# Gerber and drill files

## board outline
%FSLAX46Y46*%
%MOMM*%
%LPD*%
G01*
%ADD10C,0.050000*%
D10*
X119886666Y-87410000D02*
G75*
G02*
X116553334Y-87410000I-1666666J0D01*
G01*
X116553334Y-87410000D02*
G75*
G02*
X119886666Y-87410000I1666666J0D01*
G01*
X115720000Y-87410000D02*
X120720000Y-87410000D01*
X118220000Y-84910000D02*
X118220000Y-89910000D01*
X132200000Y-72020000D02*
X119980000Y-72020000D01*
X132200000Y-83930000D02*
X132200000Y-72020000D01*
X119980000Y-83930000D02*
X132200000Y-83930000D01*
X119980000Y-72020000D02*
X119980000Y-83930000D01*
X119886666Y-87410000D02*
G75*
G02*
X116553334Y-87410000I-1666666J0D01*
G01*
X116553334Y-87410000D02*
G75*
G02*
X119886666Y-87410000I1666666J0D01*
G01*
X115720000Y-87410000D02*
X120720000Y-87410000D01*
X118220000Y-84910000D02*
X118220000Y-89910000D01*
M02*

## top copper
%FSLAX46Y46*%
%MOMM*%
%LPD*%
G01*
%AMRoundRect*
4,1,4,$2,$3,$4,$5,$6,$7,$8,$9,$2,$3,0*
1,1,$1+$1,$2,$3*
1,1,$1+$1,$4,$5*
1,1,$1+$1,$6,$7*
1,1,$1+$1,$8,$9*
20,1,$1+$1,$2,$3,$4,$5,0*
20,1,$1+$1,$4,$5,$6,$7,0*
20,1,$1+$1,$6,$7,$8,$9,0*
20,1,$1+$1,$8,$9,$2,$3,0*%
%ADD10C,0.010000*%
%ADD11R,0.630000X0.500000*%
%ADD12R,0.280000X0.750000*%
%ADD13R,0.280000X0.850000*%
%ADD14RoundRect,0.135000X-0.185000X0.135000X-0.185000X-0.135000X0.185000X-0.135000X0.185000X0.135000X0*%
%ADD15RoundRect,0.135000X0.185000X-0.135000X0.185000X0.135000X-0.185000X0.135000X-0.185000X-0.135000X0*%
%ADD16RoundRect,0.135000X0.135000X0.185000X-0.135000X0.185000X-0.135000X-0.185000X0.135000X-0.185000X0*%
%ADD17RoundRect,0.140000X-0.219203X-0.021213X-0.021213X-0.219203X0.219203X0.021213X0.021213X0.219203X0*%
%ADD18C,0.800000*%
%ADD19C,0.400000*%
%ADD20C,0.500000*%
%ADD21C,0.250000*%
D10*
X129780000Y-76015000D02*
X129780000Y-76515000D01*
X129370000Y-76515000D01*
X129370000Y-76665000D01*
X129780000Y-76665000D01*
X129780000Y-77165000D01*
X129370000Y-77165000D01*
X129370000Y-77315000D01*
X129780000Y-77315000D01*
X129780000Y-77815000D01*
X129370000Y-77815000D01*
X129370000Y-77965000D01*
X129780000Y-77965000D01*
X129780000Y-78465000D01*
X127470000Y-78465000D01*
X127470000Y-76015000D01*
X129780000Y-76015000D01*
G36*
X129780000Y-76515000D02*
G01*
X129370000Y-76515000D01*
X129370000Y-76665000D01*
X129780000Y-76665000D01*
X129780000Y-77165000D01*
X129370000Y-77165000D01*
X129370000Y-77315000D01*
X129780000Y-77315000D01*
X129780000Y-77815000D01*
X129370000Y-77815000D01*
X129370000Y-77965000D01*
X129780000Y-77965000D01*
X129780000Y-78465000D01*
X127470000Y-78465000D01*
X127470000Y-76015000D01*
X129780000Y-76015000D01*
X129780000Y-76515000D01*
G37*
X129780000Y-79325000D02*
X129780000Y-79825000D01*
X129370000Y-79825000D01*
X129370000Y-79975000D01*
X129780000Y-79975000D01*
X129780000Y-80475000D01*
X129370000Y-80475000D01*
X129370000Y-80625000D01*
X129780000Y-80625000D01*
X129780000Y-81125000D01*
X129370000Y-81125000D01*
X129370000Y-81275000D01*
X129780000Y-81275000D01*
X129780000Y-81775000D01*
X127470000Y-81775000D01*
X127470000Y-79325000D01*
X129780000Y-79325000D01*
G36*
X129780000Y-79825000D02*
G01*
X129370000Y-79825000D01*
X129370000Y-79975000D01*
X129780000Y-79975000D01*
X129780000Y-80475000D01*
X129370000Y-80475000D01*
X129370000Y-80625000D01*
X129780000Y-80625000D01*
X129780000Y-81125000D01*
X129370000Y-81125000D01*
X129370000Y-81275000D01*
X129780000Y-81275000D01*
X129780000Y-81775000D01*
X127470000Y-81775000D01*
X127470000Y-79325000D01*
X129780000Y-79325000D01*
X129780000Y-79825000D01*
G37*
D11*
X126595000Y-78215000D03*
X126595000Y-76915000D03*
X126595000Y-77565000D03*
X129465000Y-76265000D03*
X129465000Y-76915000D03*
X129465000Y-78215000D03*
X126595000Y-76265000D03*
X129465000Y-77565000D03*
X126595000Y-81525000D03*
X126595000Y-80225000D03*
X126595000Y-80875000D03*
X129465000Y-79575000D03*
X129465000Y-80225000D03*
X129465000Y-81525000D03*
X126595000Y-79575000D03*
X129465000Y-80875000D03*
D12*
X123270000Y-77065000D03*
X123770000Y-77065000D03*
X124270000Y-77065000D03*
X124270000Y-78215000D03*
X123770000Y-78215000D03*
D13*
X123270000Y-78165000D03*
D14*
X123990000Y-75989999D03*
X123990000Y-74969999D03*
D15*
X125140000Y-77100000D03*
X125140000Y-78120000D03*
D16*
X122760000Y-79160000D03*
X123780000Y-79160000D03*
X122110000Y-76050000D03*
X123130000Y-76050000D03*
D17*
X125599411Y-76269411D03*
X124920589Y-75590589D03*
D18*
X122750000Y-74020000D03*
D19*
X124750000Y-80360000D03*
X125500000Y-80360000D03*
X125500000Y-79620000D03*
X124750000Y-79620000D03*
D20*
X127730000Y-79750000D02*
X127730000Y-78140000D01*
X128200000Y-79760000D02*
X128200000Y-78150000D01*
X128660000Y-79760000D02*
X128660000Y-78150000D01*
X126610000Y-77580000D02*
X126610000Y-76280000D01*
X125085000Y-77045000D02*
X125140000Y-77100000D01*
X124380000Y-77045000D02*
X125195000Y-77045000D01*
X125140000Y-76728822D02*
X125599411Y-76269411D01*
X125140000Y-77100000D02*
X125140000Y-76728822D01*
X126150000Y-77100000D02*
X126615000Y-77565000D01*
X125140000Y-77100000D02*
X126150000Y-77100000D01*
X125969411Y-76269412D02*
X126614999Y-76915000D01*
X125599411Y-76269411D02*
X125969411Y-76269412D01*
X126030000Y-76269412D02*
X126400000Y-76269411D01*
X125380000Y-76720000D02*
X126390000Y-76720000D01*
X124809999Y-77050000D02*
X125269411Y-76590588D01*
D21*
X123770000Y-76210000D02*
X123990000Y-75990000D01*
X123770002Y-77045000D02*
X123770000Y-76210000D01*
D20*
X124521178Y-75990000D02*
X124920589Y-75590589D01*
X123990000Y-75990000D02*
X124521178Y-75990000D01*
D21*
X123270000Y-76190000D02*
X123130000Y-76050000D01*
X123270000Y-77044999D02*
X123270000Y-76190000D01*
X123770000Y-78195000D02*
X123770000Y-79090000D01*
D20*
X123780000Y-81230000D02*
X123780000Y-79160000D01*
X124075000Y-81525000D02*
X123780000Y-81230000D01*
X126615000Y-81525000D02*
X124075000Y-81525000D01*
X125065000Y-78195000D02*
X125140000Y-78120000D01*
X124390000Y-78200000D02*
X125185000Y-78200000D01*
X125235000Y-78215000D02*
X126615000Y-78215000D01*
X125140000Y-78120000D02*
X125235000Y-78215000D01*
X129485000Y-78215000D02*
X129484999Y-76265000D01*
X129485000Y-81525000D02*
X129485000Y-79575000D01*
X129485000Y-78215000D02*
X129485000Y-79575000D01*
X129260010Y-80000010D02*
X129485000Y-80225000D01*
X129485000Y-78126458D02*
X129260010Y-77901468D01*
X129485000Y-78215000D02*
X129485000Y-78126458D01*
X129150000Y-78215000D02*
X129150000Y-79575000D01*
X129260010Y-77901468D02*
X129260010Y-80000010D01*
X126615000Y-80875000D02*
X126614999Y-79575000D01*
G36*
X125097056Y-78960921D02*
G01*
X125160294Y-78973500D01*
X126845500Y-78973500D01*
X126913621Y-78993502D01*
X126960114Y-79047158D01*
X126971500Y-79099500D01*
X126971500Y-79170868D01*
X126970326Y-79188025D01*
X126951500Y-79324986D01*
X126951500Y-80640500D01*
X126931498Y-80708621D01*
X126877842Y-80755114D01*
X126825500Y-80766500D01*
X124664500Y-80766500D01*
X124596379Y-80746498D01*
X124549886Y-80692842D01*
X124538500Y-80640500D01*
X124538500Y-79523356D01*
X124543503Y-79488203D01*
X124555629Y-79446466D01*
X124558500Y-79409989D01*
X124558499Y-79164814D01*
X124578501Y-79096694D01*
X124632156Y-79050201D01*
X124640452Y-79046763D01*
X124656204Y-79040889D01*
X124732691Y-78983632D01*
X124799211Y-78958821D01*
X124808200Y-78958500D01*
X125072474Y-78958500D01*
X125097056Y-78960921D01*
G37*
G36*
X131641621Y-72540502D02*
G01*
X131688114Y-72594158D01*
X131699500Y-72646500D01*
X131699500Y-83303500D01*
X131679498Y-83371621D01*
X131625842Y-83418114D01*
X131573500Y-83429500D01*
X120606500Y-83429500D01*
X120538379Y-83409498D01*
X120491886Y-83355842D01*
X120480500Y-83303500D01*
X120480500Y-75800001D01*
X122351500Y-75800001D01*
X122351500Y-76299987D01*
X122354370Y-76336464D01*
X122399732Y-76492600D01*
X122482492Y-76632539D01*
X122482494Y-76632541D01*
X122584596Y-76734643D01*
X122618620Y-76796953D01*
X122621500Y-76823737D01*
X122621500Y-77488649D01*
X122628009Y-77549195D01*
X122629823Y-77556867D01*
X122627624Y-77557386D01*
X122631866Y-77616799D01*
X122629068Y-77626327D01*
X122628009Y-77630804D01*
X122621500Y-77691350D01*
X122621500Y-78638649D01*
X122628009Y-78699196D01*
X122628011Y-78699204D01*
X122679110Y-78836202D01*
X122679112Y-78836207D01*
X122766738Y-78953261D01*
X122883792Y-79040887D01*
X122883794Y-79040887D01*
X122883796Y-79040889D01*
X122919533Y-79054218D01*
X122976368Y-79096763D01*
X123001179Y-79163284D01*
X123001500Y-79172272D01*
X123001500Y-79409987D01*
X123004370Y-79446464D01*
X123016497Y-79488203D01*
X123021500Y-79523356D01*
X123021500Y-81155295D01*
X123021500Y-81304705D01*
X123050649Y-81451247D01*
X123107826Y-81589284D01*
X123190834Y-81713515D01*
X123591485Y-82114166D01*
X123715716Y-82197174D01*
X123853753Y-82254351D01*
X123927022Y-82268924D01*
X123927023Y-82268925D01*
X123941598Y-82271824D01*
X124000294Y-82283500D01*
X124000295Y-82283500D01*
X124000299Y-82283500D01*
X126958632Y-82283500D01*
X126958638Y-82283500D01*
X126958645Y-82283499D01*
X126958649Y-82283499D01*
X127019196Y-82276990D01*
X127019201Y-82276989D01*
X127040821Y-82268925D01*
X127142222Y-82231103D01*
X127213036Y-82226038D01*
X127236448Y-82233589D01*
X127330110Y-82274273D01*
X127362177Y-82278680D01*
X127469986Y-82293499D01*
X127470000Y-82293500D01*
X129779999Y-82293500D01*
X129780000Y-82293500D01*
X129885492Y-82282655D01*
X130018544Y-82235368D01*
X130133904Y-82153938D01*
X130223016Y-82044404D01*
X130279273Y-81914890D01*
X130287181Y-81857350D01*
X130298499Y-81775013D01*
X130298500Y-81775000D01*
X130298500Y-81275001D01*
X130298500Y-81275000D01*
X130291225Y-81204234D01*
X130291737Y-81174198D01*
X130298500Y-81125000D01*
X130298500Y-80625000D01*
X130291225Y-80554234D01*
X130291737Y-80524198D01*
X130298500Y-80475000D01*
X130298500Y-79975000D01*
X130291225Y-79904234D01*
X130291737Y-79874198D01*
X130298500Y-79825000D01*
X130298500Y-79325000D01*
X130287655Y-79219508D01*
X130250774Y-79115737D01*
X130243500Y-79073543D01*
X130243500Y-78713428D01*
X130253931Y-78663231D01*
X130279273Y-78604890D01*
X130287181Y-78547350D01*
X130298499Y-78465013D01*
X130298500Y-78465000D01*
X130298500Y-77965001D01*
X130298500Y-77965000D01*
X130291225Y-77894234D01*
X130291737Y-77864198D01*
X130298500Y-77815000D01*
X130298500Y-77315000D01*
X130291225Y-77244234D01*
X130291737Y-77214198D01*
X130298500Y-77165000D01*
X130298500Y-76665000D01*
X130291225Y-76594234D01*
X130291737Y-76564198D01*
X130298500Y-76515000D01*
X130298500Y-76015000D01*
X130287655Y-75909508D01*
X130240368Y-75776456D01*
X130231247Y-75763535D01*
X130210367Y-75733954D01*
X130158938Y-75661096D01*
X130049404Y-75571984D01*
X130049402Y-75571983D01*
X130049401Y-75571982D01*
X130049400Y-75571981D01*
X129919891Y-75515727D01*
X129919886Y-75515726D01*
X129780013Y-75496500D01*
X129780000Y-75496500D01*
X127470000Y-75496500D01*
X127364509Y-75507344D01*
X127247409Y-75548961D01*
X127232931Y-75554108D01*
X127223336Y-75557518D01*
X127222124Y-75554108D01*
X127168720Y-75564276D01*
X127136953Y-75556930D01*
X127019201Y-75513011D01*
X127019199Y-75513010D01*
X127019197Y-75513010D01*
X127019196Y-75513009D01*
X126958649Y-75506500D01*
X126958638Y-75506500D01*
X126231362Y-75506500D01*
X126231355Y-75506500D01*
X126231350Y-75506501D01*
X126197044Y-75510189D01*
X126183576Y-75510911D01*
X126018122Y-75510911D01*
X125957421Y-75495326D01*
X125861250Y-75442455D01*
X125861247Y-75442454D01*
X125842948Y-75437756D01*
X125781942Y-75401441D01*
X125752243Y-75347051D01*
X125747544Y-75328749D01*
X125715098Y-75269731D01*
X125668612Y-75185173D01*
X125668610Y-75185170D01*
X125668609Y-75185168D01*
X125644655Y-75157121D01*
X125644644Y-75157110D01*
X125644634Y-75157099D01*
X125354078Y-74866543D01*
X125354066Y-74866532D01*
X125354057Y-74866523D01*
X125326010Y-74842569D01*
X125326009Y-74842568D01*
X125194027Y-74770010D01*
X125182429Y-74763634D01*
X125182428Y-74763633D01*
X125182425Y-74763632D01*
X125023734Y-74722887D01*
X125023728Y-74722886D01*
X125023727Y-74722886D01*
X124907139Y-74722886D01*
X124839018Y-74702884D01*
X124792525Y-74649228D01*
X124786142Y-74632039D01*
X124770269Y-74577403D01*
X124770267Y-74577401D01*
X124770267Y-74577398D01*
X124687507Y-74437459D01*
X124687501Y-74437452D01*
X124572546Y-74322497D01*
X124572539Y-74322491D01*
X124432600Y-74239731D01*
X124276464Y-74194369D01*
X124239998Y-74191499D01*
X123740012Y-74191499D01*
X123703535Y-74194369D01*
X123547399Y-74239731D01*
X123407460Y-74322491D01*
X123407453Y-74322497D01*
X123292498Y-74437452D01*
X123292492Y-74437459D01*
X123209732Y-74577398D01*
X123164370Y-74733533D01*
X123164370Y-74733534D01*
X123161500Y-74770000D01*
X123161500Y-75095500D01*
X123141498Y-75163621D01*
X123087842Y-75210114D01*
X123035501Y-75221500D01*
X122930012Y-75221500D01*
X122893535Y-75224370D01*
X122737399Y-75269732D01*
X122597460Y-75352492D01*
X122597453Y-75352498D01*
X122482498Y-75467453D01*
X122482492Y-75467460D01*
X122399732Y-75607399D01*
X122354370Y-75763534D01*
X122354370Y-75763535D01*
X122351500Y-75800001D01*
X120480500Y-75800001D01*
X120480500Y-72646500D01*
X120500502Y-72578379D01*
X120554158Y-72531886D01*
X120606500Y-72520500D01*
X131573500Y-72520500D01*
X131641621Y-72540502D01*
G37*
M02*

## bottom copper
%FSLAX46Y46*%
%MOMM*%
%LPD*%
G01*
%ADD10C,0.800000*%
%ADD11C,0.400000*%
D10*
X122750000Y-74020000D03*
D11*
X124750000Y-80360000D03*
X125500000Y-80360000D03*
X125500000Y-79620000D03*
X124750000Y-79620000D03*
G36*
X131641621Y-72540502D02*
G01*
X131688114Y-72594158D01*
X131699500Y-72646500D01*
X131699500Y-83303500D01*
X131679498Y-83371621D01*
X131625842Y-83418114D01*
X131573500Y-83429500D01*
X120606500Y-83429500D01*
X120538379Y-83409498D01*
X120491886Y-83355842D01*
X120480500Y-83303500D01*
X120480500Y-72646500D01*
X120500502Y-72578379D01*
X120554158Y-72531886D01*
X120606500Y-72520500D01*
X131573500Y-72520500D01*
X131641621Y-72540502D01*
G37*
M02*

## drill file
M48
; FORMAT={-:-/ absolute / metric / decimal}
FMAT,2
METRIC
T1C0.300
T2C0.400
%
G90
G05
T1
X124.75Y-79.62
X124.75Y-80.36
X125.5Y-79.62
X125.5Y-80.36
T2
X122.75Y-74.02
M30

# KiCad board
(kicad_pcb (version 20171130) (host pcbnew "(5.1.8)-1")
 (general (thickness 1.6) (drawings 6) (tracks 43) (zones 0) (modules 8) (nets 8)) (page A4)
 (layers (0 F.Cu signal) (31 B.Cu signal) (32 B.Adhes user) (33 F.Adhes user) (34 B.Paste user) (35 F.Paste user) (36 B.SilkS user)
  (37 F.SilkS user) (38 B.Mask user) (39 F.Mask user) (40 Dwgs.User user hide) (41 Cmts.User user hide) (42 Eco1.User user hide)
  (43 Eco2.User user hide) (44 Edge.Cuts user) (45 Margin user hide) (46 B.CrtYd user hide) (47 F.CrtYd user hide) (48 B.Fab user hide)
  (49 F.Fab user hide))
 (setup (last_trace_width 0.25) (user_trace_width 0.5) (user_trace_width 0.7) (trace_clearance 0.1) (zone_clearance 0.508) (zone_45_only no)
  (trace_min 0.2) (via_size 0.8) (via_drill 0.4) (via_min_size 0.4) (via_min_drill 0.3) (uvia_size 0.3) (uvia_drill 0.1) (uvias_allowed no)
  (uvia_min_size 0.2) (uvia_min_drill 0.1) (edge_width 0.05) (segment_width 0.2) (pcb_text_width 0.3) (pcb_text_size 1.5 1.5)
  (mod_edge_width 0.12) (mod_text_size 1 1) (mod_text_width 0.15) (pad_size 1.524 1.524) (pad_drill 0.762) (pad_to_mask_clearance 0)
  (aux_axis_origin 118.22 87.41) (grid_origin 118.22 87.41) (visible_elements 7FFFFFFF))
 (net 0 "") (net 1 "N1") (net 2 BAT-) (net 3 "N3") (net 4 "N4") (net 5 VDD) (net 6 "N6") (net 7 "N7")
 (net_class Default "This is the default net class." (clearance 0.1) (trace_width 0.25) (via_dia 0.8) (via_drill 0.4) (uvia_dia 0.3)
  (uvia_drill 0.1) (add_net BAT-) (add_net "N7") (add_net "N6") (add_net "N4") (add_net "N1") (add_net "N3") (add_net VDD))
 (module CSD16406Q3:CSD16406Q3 (layer F.Cu) (at 128.29 74.07)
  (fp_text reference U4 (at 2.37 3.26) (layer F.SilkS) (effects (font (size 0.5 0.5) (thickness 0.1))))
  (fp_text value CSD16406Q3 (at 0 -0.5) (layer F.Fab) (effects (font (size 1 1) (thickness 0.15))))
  (fp_poly
   (pts (xy 1.49 1.945) (xy 1.49 2.445) (xy 1.08 2.445) (xy 1.08 2.595) (xy 1.49 2.595) (xy 1.49 3.095) (xy 1.08 3.095) (xy 1.08 3.245)
    (xy 1.49 3.245) (xy 1.49 3.745) (xy 1.08 3.745) (xy 1.08 3.895) (xy 1.49 3.895) (xy 1.49 4.395) (xy -0.82 4.395) (xy -0.82 1.945))
   (layer F.Cu) (width 0.01))
  (pad 4 smd rect (at -1.695 4.145) (size 0.63 0.5) (layers F.Cu F.Mask) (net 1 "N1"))
  (pad 2 smd rect (at -1.695 2.845) (size 0.63 0.5) (layers F.Cu F.Mask) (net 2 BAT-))
  (pad 3 smd rect (at -1.695 3.495) (size 0.63 0.5) (layers F.Cu F.Mask) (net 2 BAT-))
  (pad 8 smd rect (at 1.175 2.195) (size 0.63 0.5) (layers F.Cu) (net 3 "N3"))
  (pad 7 smd rect (at 1.175 2.845) (size 0.63 0.5) (layers F.Cu) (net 3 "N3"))
  (pad 5 smd rect (at 1.175 4.145) (size 0.63 0.5) (layers F.Cu) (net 3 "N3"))
  (pad 1 smd rect (at -1.695 2.195) (size 0.63 0.5) (layers F.Cu F.Mask) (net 2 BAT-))
  (pad 6 smd rect (at 1.175 3.495) (size 0.63 0.5) (layers F.Cu) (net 3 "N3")))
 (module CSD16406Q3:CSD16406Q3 (layer F.Cu) (at 128.29 77.38)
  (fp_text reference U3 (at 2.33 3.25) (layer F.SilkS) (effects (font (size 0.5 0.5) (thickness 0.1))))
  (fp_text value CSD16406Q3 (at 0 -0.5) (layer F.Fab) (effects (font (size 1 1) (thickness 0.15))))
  (fp_poly
   (pts (xy 1.49 1.945) (xy 1.49 2.445) (xy 1.08 2.445) (xy 1.08 2.595) (xy 1.49 2.595) (xy 1.49 3.095) (xy 1.08 3.095) (xy 1.08 3.245)
    (xy 1.49 3.245) (xy 1.49 3.745) (xy 1.08 3.745) (xy 1.08 3.895) (xy 1.49 3.895) (xy 1.49 4.395) (xy -0.82 4.395) (xy -0.82 1.945))
   (layer F.Cu) (width 0.01))
  (pad 4 smd rect (at -1.695 4.145) (size 0.63 0.5) (layers F.Cu F.Mask) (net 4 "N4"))
  (pad 2 smd rect (at -1.695 2.845) (size 0.63 0.5) (layers F.Cu F.Mask) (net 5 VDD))
  (pad 3 smd rect (at -1.695 3.495) (size 0.63 0.5) (layers F.Cu F.Mask) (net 5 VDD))
  (pad 8 smd rect (at 1.175 2.195) (size 0.63 0.5) (layers F.Cu) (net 3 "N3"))
  (pad 7 smd rect (at 1.175 2.845) (size 0.63 0.5) (layers F.Cu) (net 3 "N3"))
  (pad 5 smd rect (at 1.175 4.145) (size 0.63 0.5) (layers F.Cu) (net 3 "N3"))
  (pad 1 smd rect (at -1.695 2.195) (size 0.63 0.5) (layers F.Cu F.Mask) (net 5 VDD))
  (pad 6 smd rect (at 1.175 3.495) (size 0.63 0.5) (layers F.Cu) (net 3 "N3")))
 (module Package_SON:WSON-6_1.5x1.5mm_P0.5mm (layer F.Cu) (at 123.77 77.64 90)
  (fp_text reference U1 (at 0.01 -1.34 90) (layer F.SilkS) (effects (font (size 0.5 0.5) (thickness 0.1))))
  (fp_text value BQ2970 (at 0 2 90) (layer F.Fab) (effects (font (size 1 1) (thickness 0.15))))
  (pad 6 smd rect (at 0.575 -0.5) (size 0.28 0.75) (layers F.Cu F.Paste F.Mask) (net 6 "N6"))
  (pad 5 smd rect (at 0.575 0) (size 0.28 0.75) (layers F.Cu F.Paste F.Mask) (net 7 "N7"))
  (pad 4 smd rect (at 0.575 0.5) (size 0.28 0.75) (layers F.Cu F.Paste F.Mask) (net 2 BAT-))
  (pad 3 smd rect (at -0.575 0.5) (size 0.28 0.75) (layers F.Cu F.Paste F.Mask) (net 1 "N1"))
  (pad 2 smd rect (at -0.575 0) (size 0.28 0.75) (layers F.Cu F.Paste F.Mask) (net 4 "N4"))
  (pad 1 smd rect (at -0.525 -0.5) (size 0.28 0.85) (layers F.Cu F.Paste F.Mask)))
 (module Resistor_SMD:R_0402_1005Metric (layer F.Cu) (at 123.99 75.479999 270)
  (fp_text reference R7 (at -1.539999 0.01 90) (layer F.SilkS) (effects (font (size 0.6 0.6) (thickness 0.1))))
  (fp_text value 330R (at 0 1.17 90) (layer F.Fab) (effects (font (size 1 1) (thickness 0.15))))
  (pad 2 smd roundrect (at 0.51 0 270) (size 0.54 0.64) (layers F.Cu F.Paste F.Mask) (roundrect_rratio 0.25) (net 7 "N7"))
  (pad 1 smd roundrect (at -0.51 0 270) (size 0.54 0.64) (layers F.Cu F.Paste F.Mask) (roundrect_rratio 0.25)))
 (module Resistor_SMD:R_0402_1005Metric (layer F.Cu) (at 125.14 77.61 90)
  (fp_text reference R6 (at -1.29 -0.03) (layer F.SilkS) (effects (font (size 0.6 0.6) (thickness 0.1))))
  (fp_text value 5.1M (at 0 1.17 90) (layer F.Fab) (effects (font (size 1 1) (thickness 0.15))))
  (pad 2 smd roundrect (at 0.51 0 90) (size 0.54 0.64) (layers F.Cu F.Paste F.Mask) (roundrect_rratio 0.25) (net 2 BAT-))
  (pad 1 smd roundrect (at -0.51 0 90) (size 0.54 0.64) (layers F.Cu F.Paste F.Mask) (roundrect_rratio 0.25) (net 1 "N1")))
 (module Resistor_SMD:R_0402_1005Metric (layer F.Cu) (at 123.27 79.16 180)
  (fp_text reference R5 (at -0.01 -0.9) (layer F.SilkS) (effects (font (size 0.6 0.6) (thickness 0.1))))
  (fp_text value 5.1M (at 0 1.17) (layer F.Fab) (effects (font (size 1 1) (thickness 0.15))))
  (pad 2 smd roundrect (at 0.51 0 180) (size 0.54 0.64) (layers F.Cu F.Paste F.Mask) (roundrect_rratio 0.25) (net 5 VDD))
  (pad 1 smd roundrect (at -0.51 0 180) (size 0.54 0.64) (layers F.Cu F.Paste F.Mask) (roundrect_rratio 0.25) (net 4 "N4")))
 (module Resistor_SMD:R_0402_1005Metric (layer F.Cu) (at 122.62 76.05 180)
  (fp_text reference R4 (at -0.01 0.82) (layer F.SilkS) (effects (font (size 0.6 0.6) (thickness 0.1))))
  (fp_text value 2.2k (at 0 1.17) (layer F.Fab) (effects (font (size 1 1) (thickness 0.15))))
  (pad 2 smd roundrect (at 0.51 0 180) (size 0.54 0.64) (layers F.Cu F.Paste F.Mask) (roundrect_rratio 0.25) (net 5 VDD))
  (pad 1 smd roundrect (at -0.51 0 180) (size 0.54 0.64) (layers F.Cu F.Paste F.Mask) (roundrect_rratio 0.25) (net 6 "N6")))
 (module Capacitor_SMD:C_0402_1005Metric (layer F.Cu) (at 125.26 75.93 315)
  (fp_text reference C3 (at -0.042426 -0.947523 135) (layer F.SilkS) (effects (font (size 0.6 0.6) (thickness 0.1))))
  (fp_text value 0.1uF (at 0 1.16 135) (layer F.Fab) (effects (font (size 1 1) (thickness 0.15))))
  (pad 2 smd roundrect (at 0.48 0 315) (size 0.56 0.62) (layers F.Cu F.Paste F.Mask) (roundrect_rratio 0.25) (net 2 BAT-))
  (pad 1 smd roundrect (at -0.48 0 315) (size 0.56 0.62) (layers F.Cu F.Paste F.Mask) (roundrect_rratio 0.25) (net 7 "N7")))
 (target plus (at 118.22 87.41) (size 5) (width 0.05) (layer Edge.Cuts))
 (gr_line (start 132.2 72.02) (end 119.98 72.02) (layer Edge.Cuts) (width 0.05))
 (gr_line (start 132.2 83.93) (end 132.2 72.02) (layer Edge.Cuts) (width 0.05))
 (gr_line (start 119.98 83.93) (end 132.2 83.93) (layer Edge.Cuts) (width 0.05))
 (gr_line (start 119.98 72.02) (end 119.98 83.93) (layer Edge.Cuts) (width 0.05))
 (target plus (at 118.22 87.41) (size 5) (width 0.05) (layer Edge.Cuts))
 (segment (start 127.73 79.75) (end 127.73 78.14) (width 0.5) (layer F.Cu) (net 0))
 (segment (start 128.2 79.76) (end 128.2 78.15) (width 0.5) (layer F.Cu) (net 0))
 (segment (start 128.66 79.76) (end 128.66 78.15) (width 0.5) (layer F.Cu) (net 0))
 (segment (start 126.61 77.58) (end 126.61 76.28) (width 0.5) (layer F.Cu) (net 2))
 (segment (start 125.085 77.045) (end 125.14 77.1) (width 0.5) (layer F.Cu) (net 2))
 (segment (start 124.38 77.045) (end 125.195 77.045) (width 0.5) (layer F.Cu) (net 2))
 (segment (start 125.14 76.728822) (end 125.599411 76.269411) (width 0.5) (layer F.Cu) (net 2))
 (segment (start 125.14 77.1) (end 125.14 76.728822) (width 0.5) (layer F.Cu) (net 2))
 (segment (start 126.15 77.1) (end 126.615 77.565) (width 0.5) (layer F.Cu) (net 2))
 (segment (start 125.14 77.1) (end 126.15 77.1) (width 0.5) (layer F.Cu) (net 2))
 (segment (start 125.969411 76.269412) (end 126.614999 76.915) (width 0.5) (layer F.Cu) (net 2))
 (segment (start 125.599411 76.269411) (end 125.969411 76.269412) (width 0.5) (layer F.Cu) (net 2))
 (segment (start 126.03 76.269412) (end 126.4 76.269411) (width 0.5) (layer F.Cu) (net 2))
 (segment (start 125.38 76.72) (end 126.39 76.72) (width 0.5) (layer F.Cu) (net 2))
 (segment (start 124.809999 77.05) (end 125.269411 76.590588) (width 0.5) (layer F.Cu) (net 2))
 (segment (start 123.77 76.21) (end 123.99 75.99) (width 0.25) (layer F.Cu) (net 7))
 (segment (start 123.770002 77.045) (end 123.77 76.21) (width 0.25) (layer F.Cu) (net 7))
 (segment (start 124.521178 75.99) (end 124.920589 75.590589) (width 0.5) (layer F.Cu) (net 7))
 (segment (start 123.99 75.99) (end 124.521178 75.99) (width 0.5) (layer F.Cu) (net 7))
 (segment (start 123.27 76.19) (end 123.13 76.05) (width 0.25) (layer F.Cu) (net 6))
 (segment (start 123.27 77.044999) (end 123.27 76.19) (width 0.25) (layer F.Cu) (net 6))
 (segment (start 123.77 78.195) (end 123.77 79.09) (width 0.25) (layer F.Cu) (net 4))
 (segment (start 123.78 81.23) (end 123.78 79.16) (width 0.5) (layer F.Cu) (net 4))
 (segment (start 124.075 81.525) (end 123.78 81.23) (width 0.5) (layer F.Cu) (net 4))
 (segment (start 126.615 81.525) (end 124.075 81.525) (width 0.5) (layer F.Cu) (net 4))
 (segment (start 125.065 78.195) (end 125.14 78.12) (width 0.5) (layer F.Cu) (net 1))
 (segment (start 124.39 78.2) (end 125.185 78.2) (width 0.5) (layer F.Cu) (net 1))
 (segment (start 125.235 78.215) (end 126.615 78.215) (width 0.5) (layer F.Cu) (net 1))
 (segment (start 125.14 78.12) (end 125.235 78.215) (width 0.5) (layer F.Cu) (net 1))
 (segment (start 129.485 78.215) (end 129.484999 76.265) (width 0.5) (layer F.Cu) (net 3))
 (segment (start 129.485 81.525) (end 129.485 79.575) (width 0.5) (layer F.Cu) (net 3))
 (segment (start 129.485 78.215) (end 129.485 79.575) (width 0.5) (layer F.Cu) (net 3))
 (segment (start 129.26001 80.00001) (end 129.485 80.225) (width 0.5) (layer F.Cu) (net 3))
 (segment (start 129.485 78.126458) (end 129.26001 77.901468) (width 0.5) (layer F.Cu) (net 3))
 (segment (start 129.485 78.215) (end 129.485 78.126458) (width 0.5) (layer F.Cu) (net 3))
 (segment (start 129.15 78.215) (end 129.15 79.575) (width 0.5) (layer F.Cu) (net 3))
 (segment (start 129.26001 77.901468) (end 129.26001 80.00001) (width 0.5) (layer F.Cu) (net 3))
 (segment (start 126.615 80.875) (end 126.614999 79.575) (width 0.5) (layer F.Cu) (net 5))
 (via (at 122.75 74.02) (size 0.8) (drill 0.4) (layers F.Cu B.Cu) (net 5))
 (via (at 124.75 80.36) (size 0.4) (drill 0.3) (layers F.Cu B.Cu) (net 5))
 (via (at 125.5 80.36) (size 0.4) (drill 0.3) (layers F.Cu B.Cu) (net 5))
 (via (at 125.5 79.62) (size 0.4) (drill 0.3) (layers F.Cu B.Cu) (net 5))
 (via (at 124.75 79.62) (size 0.4) (drill 0.3) (layers F.Cu B.Cu) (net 5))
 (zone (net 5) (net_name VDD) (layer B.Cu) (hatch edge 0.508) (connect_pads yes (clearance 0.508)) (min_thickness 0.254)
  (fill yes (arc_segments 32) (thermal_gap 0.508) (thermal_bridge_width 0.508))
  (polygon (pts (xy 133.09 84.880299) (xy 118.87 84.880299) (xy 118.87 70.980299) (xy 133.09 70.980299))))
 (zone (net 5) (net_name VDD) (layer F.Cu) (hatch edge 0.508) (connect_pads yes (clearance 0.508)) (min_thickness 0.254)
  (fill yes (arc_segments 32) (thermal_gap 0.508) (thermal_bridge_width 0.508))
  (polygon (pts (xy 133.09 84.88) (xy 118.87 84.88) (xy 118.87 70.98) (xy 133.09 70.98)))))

